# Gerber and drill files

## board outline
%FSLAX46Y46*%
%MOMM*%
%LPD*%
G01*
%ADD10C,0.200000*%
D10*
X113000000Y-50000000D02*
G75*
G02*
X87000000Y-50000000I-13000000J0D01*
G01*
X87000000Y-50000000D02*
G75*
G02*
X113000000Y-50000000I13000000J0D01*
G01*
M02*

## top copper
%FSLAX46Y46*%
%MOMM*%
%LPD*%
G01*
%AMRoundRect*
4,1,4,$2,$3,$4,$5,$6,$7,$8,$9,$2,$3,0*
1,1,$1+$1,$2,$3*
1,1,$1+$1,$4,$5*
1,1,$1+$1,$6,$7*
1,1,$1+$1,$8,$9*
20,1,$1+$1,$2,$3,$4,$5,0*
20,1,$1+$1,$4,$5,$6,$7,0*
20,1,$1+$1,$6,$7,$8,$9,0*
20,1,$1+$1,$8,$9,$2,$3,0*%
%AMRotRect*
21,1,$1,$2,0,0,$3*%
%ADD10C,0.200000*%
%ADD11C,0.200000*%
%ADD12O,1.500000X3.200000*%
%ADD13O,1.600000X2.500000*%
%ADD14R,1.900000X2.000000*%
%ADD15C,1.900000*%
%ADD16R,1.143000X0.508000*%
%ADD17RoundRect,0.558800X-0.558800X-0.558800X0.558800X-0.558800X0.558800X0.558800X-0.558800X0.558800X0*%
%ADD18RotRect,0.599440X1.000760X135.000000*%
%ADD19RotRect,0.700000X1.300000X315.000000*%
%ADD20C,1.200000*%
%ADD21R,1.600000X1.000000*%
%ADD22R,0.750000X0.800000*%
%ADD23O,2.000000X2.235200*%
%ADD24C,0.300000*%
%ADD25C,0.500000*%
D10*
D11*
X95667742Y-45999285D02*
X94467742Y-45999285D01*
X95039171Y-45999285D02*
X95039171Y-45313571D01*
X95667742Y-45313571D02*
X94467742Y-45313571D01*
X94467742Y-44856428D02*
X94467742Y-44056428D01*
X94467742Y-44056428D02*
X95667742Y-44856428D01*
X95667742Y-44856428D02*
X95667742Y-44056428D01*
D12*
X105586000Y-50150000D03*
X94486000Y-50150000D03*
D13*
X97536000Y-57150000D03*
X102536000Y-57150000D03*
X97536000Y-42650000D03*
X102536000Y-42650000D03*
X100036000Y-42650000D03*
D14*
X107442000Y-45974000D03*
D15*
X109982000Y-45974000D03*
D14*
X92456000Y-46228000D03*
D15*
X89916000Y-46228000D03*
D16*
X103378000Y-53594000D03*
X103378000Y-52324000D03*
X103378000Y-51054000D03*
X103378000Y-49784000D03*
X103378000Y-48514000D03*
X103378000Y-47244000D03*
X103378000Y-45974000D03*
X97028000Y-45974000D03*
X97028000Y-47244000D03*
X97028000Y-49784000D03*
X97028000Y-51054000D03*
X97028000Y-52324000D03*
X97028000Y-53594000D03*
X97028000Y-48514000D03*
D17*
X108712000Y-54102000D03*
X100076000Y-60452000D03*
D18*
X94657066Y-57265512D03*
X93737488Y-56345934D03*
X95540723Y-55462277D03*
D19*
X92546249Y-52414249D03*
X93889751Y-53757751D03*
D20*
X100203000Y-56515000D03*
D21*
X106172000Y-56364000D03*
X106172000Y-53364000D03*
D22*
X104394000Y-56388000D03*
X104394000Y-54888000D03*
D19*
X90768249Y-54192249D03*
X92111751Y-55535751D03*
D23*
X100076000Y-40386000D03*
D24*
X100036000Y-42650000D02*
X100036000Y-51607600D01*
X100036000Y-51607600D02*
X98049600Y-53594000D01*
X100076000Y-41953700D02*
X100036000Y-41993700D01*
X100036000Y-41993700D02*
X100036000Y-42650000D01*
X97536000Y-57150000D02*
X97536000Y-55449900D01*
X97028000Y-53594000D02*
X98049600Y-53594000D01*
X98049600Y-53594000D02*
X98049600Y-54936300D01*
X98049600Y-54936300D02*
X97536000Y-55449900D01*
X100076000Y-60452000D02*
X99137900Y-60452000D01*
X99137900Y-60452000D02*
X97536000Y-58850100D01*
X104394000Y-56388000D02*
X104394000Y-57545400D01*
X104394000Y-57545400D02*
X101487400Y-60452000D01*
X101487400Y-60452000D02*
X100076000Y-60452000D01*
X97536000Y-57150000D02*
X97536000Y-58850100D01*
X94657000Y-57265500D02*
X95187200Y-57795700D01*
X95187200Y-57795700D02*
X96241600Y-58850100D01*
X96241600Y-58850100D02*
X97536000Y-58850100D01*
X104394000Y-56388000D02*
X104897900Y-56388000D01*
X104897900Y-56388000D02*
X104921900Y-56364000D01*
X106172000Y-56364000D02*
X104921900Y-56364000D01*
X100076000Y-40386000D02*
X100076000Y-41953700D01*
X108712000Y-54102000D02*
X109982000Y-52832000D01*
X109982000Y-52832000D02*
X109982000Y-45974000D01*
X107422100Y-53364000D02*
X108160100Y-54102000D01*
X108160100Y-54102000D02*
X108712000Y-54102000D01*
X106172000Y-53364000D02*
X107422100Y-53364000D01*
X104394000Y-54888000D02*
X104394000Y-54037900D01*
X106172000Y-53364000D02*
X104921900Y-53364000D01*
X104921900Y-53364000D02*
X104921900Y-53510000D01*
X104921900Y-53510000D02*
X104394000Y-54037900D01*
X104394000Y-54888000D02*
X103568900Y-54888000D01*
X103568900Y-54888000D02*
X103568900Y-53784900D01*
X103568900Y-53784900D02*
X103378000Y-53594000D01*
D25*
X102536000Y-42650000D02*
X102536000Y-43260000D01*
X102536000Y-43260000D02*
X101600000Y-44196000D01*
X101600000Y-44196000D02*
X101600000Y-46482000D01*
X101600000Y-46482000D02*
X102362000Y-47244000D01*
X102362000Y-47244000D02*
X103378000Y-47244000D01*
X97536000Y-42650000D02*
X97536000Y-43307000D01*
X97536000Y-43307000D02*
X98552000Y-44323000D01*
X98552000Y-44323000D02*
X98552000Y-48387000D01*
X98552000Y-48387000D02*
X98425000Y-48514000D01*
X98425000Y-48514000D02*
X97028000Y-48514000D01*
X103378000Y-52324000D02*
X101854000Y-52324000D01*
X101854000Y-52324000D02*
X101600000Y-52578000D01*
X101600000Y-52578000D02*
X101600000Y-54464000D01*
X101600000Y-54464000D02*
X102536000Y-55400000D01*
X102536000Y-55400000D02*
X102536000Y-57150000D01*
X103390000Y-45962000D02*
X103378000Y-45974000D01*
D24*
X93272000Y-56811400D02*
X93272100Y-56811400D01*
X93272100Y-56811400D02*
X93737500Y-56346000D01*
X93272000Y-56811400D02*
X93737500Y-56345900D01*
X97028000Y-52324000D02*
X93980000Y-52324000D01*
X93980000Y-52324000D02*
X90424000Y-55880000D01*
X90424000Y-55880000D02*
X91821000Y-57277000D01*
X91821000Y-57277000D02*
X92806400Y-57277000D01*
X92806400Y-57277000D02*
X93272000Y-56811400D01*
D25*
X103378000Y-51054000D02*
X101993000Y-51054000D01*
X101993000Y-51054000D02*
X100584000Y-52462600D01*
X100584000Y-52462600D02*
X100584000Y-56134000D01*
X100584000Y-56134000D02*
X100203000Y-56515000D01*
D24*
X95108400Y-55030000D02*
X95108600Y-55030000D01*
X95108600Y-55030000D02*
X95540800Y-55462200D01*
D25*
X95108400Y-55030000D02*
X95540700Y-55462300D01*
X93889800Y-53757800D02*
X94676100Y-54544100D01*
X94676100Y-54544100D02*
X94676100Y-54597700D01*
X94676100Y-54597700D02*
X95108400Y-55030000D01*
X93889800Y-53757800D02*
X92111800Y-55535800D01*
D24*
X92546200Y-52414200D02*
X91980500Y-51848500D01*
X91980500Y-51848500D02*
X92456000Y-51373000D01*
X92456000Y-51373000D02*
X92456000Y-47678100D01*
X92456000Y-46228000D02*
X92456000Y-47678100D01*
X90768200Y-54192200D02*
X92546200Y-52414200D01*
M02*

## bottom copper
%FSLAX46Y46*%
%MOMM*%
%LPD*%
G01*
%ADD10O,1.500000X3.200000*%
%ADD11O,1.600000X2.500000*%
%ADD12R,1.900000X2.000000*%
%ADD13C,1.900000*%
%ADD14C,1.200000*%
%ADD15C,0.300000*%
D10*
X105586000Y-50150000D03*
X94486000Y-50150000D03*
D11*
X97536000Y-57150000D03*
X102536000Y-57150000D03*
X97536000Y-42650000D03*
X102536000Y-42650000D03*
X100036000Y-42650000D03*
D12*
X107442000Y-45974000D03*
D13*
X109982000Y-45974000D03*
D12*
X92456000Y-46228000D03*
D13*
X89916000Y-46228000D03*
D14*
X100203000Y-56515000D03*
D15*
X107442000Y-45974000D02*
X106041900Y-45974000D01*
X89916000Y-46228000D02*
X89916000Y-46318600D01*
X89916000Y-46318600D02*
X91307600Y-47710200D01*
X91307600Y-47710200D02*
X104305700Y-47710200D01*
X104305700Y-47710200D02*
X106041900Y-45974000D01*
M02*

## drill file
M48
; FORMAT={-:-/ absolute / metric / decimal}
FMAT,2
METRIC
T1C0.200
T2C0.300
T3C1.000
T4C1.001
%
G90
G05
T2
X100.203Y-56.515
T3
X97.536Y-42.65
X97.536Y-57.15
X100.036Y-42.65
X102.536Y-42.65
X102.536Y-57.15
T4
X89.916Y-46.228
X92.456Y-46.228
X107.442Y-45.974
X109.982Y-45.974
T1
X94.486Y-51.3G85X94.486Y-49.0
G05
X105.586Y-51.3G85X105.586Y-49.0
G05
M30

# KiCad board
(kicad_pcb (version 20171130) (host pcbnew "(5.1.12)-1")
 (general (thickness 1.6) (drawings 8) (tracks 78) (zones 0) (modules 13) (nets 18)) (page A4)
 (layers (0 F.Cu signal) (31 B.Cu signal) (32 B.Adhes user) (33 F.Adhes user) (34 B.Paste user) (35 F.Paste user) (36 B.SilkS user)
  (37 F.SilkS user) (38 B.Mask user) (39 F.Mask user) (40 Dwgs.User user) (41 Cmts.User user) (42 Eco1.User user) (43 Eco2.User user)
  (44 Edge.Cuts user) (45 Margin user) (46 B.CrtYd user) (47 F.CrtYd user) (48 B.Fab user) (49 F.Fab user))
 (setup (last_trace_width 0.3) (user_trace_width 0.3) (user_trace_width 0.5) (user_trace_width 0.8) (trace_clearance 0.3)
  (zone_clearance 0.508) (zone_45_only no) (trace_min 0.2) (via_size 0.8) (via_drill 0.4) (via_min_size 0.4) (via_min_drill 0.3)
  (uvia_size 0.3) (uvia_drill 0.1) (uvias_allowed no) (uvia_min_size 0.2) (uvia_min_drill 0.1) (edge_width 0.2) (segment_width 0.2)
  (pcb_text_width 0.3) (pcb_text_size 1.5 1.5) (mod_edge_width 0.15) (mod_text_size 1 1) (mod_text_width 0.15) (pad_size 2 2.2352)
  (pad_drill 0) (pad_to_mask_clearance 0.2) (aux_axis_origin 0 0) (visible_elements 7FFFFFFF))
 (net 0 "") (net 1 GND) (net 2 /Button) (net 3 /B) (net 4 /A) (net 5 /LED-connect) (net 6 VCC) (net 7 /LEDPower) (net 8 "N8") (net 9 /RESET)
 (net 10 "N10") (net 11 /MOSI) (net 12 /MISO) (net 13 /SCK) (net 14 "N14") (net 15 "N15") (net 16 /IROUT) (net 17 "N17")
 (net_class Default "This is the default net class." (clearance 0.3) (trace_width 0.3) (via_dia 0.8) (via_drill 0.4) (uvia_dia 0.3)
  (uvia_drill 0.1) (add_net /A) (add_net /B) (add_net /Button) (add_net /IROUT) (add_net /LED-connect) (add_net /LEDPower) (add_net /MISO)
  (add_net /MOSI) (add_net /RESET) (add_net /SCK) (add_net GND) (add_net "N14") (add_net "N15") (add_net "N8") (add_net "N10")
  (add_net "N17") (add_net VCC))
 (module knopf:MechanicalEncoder (layer B.Cu) (at 100.036 50.15 180)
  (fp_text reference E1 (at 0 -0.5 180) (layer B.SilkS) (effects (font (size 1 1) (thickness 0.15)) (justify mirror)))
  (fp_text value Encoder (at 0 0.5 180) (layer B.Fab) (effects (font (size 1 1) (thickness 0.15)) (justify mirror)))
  (pad 6 thru_hole oval (at -5.55 0 180) (size 1.5 3.2) (drill oval 0.2 2.5) (layers *.Cu *.Mask))
  (pad 6 thru_hole oval (at 5.55 0 180) (size 1.5 3.2) (drill oval 0.2 2.5) (layers *.Cu *.Mask))
  (pad 5 thru_hole oval (at 2.5 -7 180) (size 1.6 2.5) (drill 1) (layers *.Cu *.Mask) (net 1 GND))
  (pad 4 thru_hole oval (at -2.5 -7 180) (size 1.6 2.5) (drill 1) (layers *.Cu *.Mask) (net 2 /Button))
  (pad 3 thru_hole oval (at 2.5 7.5 180) (size 1.6 2.5) (drill 1) (layers *.Cu *.Mask) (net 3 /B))
  (pad 1 thru_hole oval (at -2.5 7.5 180) (size 1.6 2.5) (drill 1) (layers *.Cu *.Mask) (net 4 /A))
  (pad 2 thru_hole oval (at 0 7.5 180) (size 1.6 2.5) (drill 1) (layers *.Cu *.Mask) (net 1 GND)))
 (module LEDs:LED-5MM (layer F.Cu) (at 107.442 45.974)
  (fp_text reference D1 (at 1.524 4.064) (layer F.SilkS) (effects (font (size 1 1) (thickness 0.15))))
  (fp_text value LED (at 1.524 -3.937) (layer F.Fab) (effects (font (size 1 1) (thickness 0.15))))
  (pad 1 thru_hole rect (at 0 0 90) (size 2 1.9) (drill 1.00076) (layers *.Cu *.Mask F.SilkS) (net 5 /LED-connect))
  (pad 2 thru_hole circle (at 2.54 0) (size 1.9 1.9) (drill 1.00076) (layers *.Cu *.Mask F.SilkS) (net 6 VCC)))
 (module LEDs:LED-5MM (layer F.Cu) (at 92.456 46.228 180)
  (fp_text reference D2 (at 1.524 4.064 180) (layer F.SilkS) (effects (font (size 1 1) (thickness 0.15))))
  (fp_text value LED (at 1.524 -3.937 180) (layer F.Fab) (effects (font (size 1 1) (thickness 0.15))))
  (pad 1 thru_hole rect (at 0 0 270) (size 2 1.9) (drill 1.00076) (layers *.Cu *.Mask F.SilkS) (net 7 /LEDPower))
  (pad 2 thru_hole circle (at 2.54 0 180) (size 1.9 1.9) (drill 1.00076) (layers *.Cu *.Mask F.SilkS) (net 5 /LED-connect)))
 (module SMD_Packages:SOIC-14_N (layer F.Cu) (at 100.076 49.784 90)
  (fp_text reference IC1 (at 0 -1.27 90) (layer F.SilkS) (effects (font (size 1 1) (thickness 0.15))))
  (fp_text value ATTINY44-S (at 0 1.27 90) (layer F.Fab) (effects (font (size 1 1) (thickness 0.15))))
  (pad 1 smd rect (at -3.81 3.302 90) (size 0.508 1.143) (layers F.Cu F.Paste F.Mask) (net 6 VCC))
  (pad 2 smd rect (at -2.54 3.302 90) (size 0.508 1.143) (layers F.Cu F.Paste F.Mask) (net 2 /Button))
  (pad 3 smd rect (at -1.27 3.302 90) (size 0.508 1.143) (layers F.Cu F.Paste F.Mask) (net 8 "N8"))
  (pad 4 smd rect (at 0 3.302 90) (size 0.508 1.143) (layers F.Cu F.Paste F.Mask) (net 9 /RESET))
  (pad 5 smd rect (at 1.27 3.302 90) (size 0.508 1.143) (layers F.Cu F.Paste F.Mask) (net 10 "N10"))
  (pad 6 smd rect (at 2.54 3.302 90) (size 0.508 1.143) (layers F.Cu F.Paste F.Mask) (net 4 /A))
  (pad 7 smd rect (at 3.81 3.302 90) (size 0.508 1.143) (layers F.Cu F.Paste F.Mask) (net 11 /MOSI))
  (pad 8 smd rect (at 3.81 -3.048 90) (size 0.508 1.143) (layers F.Cu F.Paste F.Mask) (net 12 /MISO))
  (pad 9 smd rect (at 2.54 -3.048 90) (size 0.508 1.143) (layers F.Cu F.Paste F.Mask) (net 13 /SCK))
  (pad 11 smd rect (at 0 -3.048 90) (size 0.508 1.143) (layers F.Cu F.Paste F.Mask) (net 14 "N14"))
  (pad 12 smd rect (at -1.27 -3.048 90) (size 0.508 1.143) (layers F.Cu F.Paste F.Mask) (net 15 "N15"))
  (pad 13 smd rect (at -2.54 -3.048 90) (size 0.508 1.143) (layers F.Cu F.Paste F.Mask) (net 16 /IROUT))
  (pad 14 smd rect (at -3.81 -3.048 90) (size 0.508 1.143) (layers F.Cu F.Paste F.Mask) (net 1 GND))
  (pad 10 smd rect (at 1.27 -3.048 90) (size 0.508 1.143) (layers F.Cu F.Paste F.Mask) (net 3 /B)))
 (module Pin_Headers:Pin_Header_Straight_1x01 (layer F.Cu) (at 108.712 54.102)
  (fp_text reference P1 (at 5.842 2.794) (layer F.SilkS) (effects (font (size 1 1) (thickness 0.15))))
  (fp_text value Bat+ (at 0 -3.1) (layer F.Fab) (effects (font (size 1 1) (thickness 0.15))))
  (pad 1 smd roundrect (at 0 0) (size 2.2352 2.2352) (layers F.Cu F.Paste F.Mask) (roundrect_rratio 0.25) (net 6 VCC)))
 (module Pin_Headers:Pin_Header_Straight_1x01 (layer F.Cu) (at 100.076 60.452)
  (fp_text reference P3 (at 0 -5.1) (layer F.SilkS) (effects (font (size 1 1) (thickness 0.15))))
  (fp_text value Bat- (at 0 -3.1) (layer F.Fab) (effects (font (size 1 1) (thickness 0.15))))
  (pad 1 smd roundrect (at 0 0) (size 2.2352 2.2352) (layers F.Cu F.Paste F.Mask) (roundrect_rratio 0.25) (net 1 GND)))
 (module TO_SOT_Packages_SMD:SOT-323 (layer F.Cu) (at 94.869 56.134 135)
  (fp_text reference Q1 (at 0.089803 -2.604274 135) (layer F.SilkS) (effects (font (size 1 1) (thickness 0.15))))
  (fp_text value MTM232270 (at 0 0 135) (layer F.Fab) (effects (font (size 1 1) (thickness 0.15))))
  (pad 2 smd rect (at -0.65024 -0.94996 135) (size 0.59944 1.00076) (layers F.Cu F.Paste F.Mask) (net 1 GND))
  (pad 1 smd rect (at 0.65024 -0.94996 135) (size 0.59944 1.00076) (layers F.Cu F.Paste F.Mask) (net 16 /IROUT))
  (pad 3 smd rect (at 0 0.94996 135) (size 0.59944 1.00076) (layers F.Cu F.Paste F.Mask) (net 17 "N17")))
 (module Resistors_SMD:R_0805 (layer F.Cu) (at 93.218 53.086 315)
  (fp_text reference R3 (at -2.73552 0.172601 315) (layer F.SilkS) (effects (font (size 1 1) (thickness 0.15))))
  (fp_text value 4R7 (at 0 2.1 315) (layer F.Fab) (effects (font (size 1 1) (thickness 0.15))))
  (pad 1 smd rect (at -0.949999 0 315) (size 0.7 1.3) (layers F.Cu F.Paste F.Mask) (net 7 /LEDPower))
  (pad 2 smd rect (at 0.949999 0 315) (size 0.7 1.3) (layers F.Cu F.Paste F.Mask) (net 17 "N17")))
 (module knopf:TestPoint (layer F.Cu) (at 100.203 56.515)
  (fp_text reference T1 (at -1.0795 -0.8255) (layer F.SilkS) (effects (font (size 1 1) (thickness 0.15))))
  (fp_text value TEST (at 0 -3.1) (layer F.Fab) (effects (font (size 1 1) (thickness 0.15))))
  (pad 1 thru_hole circle (at 0 0) (size 1.2 1.2) (drill 0.3) (layers *.Cu *.Mask F.SilkS) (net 8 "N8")))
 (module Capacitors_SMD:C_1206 (layer F.Cu) (at 106.172 54.864 270)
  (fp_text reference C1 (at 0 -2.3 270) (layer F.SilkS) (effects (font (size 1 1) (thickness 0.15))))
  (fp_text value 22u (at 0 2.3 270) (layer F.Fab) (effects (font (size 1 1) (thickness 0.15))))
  (pad 2 smd rect (at 1.5 0 270) (size 1 1.6) (layers F.Cu F.Paste F.Mask) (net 1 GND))
  (pad 1 smd rect (at -1.5 0 270) (size 1 1.6) (layers F.Cu F.Paste F.Mask) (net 6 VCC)))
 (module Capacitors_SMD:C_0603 (layer F.Cu) (at 104.394 55.638 270)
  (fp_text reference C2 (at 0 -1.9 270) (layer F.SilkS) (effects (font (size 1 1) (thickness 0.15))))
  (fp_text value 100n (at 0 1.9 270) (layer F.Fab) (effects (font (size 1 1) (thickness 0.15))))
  (pad 2 smd rect (at 0.75 0 270) (size 0.8 0.75) (layers F.Cu F.Paste F.Mask) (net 1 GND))
  (pad 1 smd rect (at -0.75 0 270) (size 0.8 0.75) (layers F.Cu F.Paste F.Mask) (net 6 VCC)))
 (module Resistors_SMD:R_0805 (layer F.Cu) (at 91.44 54.864 315)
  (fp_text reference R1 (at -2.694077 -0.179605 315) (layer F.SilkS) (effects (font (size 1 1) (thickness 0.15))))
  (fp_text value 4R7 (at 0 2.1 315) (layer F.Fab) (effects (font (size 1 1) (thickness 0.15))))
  (pad 1 smd rect (at -0.949999 0 315) (size 0.7 1.3) (layers F.Cu F.Paste F.Mask) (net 7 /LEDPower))
  (pad 2 smd rect (at 0.949999 0 315) (size 0.7 1.3) (layers F.Cu F.Paste F.Mask) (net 17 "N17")))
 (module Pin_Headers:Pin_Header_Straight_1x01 (layer F.Cu) (at 100.076 40.386)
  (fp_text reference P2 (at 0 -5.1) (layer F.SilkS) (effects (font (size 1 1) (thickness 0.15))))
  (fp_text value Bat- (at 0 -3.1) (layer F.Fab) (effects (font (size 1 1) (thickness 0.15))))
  (pad 1 smd oval (at 0 0) (size 2 2.2352) (layers F.Cu F.Paste F.Mask) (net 1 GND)))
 (gr_circle (center 100 50) (end 113 50) (layer Edge.Cuts) (width 0.2))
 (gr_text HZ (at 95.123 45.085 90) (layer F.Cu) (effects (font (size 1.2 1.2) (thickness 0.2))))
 (segment (start 100.036 42.65) (end 100.036 51.6076) (width 0.3) (layer F.Cu) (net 1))
 (segment (start 100.036 51.6076) (end 98.0496 53.594) (width 0.3) (layer F.Cu) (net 1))
 (segment (start 100.076 41.9537) (end 100.036 41.9937) (width 0.3) (layer F.Cu) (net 1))
 (segment (start 100.036 41.9937) (end 100.036 42.65) (width 0.3) (layer F.Cu) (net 1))
 (segment (start 97.536 57.15) (end 97.536 55.4499) (width 0.3) (layer F.Cu) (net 1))
 (segment (start 97.028 53.594) (end 98.0496 53.594) (width 0.3) (layer F.Cu) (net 1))
 (segment (start 98.0496 53.594) (end 98.0496 54.9363) (width 0.3) (layer F.Cu) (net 1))
 (segment (start 98.0496 54.9363) (end 97.536 55.4499) (width 0.3) (layer F.Cu) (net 1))
 (segment (start 100.076 60.452) (end 99.1379 60.452) (width 0.3) (layer F.Cu) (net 1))
 (segment (start 99.1379 60.452) (end 97.536 58.8501) (width 0.3) (layer F.Cu) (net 1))
 (segment (start 104.394 56.388) (end 104.394 57.5454) (width 0.3) (layer F.Cu) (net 1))
 (segment (start 104.394 57.5454) (end 101.4874 60.452) (width 0.3) (layer F.Cu) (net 1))
 (segment (start 101.4874 60.452) (end 100.076 60.452) (width 0.3) (layer F.Cu) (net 1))
 (segment (start 97.536 57.15) (end 97.536 58.8501) (width 0.3) (layer F.Cu) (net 1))
 (segment (start 94.657 57.2655) (end 95.1872 57.7957) (width 0.3) (layer F.Cu) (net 1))
 (segment (start 95.1872 57.7957) (end 96.2416 58.8501) (width 0.3) (layer F.Cu) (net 1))
 (segment (start 96.2416 58.8501) (end 97.536 58.8501) (width 0.3) (layer F.Cu) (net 1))
 (segment (start 104.394 56.388) (end 104.8979 56.388) (width 0.3) (layer F.Cu) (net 1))
 (segment (start 104.8979 56.388) (end 104.9219 56.364) (width 0.3) (layer F.Cu) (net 1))
 (segment (start 106.172 56.364) (end 104.9219 56.364) (width 0.3) (layer F.Cu) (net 1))
 (segment (start 100.076 40.386) (end 100.076 41.9537) (width 0.3) (layer F.Cu) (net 1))
 (segment (start 108.712 54.102) (end 109.982 52.832) (width 0.3) (layer F.Cu) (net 6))
 (segment (start 109.982 52.832) (end 109.982 45.974) (width 0.3) (layer F.Cu) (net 6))
 (segment (start 107.4221 53.364) (end 108.1601 54.102) (width 0.3) (layer F.Cu) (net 6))
 (segment (start 108.1601 54.102) (end 108.712 54.102) (width 0.3) (layer F.Cu) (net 6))
 (segment (start 106.172 53.364) (end 107.4221 53.364) (width 0.3) (layer F.Cu) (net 6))
 (segment (start 104.394 54.888) (end 104.394 54.0379) (width 0.3) (layer F.Cu) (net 6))
 (segment (start 106.172 53.364) (end 104.9219 53.364) (width 0.3) (layer F.Cu) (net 6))
 (segment (start 104.9219 53.364) (end 104.9219 53.51) (width 0.3) (layer F.Cu) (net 6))
 (segment (start 104.9219 53.51) (end 104.394 54.0379) (width 0.3) (layer F.Cu) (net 6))
 (segment (start 104.394 54.888) (end 103.5689 54.888) (width 0.3) (layer F.Cu) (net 6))
 (segment (start 103.5689 54.888) (end 103.5689 53.7849) (width 0.3) (layer F.Cu) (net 6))
 (segment (start 103.5689 53.7849) (end 103.378 53.594) (width 0.3) (layer F.Cu) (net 6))
 (segment (start 102.536 42.65) (end 102.536 43.26) (width 0.5) (layer F.Cu) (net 4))
 (segment (start 102.536 43.26) (end 101.6 44.196) (width 0.5) (layer F.Cu) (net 4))
 (segment (start 101.6 44.196) (end 101.6 46.482) (width 0.5) (layer F.Cu) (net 4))
 (segment (start 101.6 46.482) (end 102.362 47.244) (width 0.5) (layer F.Cu) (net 4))
 (segment (start 102.362 47.244) (end 103.378 47.244) (width 0.5) (layer F.Cu) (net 4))
 (segment (start 97.536 42.65) (end 97.536 43.307) (width 0.5) (layer F.Cu) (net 3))
 (segment (start 97.536 43.307) (end 98.552 44.323) (width 0.5) (layer F.Cu) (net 3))
 (segment (start 98.552 44.323) (end 98.552 48.387) (width 0.5) (layer F.Cu) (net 3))
 (segment (start 98.552 48.387) (end 98.425 48.514) (width 0.5) (layer F.Cu) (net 3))
 (segment (start 98.425 48.514) (end 97.028 48.514) (width 0.5) (layer F.Cu) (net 3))
 (segment (start 103.378 52.324) (end 101.854 52.324) (width 0.5) (layer F.Cu) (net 2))
 (segment (start 101.854 52.324) (end 101.6 52.578) (width 0.5) (layer F.Cu) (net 2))
 (segment (start 101.6 52.578) (end 101.6 54.464) (width 0.5) (layer F.Cu) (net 2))
 (segment (start 101.6 54.464) (end 102.536 55.4) (width 0.5) (layer F.Cu) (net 2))
 (segment (start 102.536 55.4) (end 102.536 57.15) (width 0.5) (layer F.Cu) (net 2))
 (segment (start 103.39 45.962) (end 103.378 45.974) (width 0.5) (layer F.Cu) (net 11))
 (segment (start 93.272 56.8114) (end 93.2721 56.8114) (width 0.3) (layer F.Cu) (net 16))
 (segment (start 93.2721 56.8114) (end 93.7375 56.346) (width 0.3) (layer F.Cu) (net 16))
 (segment (start 93.272 56.8114) (end 93.7375 56.3459) (width 0.3) (layer F.Cu) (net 16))
 (segment (start 97.028 52.324) (end 93.98 52.324) (width 0.3) (layer F.Cu) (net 16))
 (segment (start 93.98 52.324) (end 90.424 55.88) (width 0.3) (layer F.Cu) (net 16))
 (segment (start 90.424 55.88) (end 91.821 57.277) (width 0.3) (layer F.Cu) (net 16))
 (segment (start 91.821 57.277) (end 92.8064 57.277) (width 0.3) (layer F.Cu) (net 16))
 (segment (start 92.8064 57.277) (end 93.272 56.8114) (width 0.3) (layer F.Cu) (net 16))
 (segment (start 103.378 51.054) (end 101.993 51.054) (width 0.5) (layer F.Cu) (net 8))
 (segment (start 101.993 51.054) (end 100.584 52.4626) (width 0.5) (layer F.Cu) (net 8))
 (segment (start 100.584 52.4626) (end 100.584 56.134) (width 0.5) (layer F.Cu) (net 8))
 (segment (start 100.584 56.134) (end 100.203 56.515) (width 0.5) (layer F.Cu) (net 8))
 (segment (start 95.1084 55.03) (end 95.1086 55.03) (width 0.3) (layer F.Cu) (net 17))
 (segment (start 95.1086 55.03) (end 95.5408 55.4622) (width 0.3) (layer F.Cu) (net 17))
 (segment (start 95.1084 55.03) (end 95.5407 55.4623) (width 0.5) (layer F.Cu) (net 17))
 (segment (start 93.8898 53.7578) (end 94.6761 54.5441) (width 0.5) (layer F.Cu) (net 17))
 (segment (start 94.6761 54.5441) (end 94.6761 54.5977) (width 0.5) (layer F.Cu) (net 17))
 (segment (start 94.6761 54.5977) (end 95.1084 55.03) (width 0.5) (layer F.Cu) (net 17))
 (segment (start 93.8898 53.7578) (end 92.1118 55.5358) (width 0.5) (layer F.Cu) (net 17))
 (segment (start 107.442 45.974) (end 106.0419 45.974) (width 0.3) (layer B.Cu) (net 5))
 (segment (start 89.916 46.228) (end 89.916 46.3186) (width 0.3) (layer B.Cu) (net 5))
 (segment (start 89.916 46.3186) (end 91.3076 47.7102) (width 0.3) (layer B.Cu) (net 5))
 (segment (start 91.3076 47.7102) (end 104.3057 47.7102) (width 0.3) (layer B.Cu) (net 5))
 (segment (start 104.3057 47.7102) (end 106.0419 45.974) (width 0.3) (layer B.Cu) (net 5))
 (segment (start 92.5462 52.4142) (end 91.9805 51.8485) (width 0.3) (layer F.Cu) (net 7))
 (segment (start 91.9805 51.8485) (end 92.456 51.373) (width 0.3) (layer F.Cu) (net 7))
 (segment (start 92.456 51.373) (end 92.456 47.6781) (width 0.3) (layer F.Cu) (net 7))
 (segment (start 92.456 46.228) (end 92.456 47.6781) (width 0.3) (layer F.Cu) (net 7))
 (segment (start 90.7682 54.1922) (end 92.5462 52.4142) (width 0.3) (layer F.Cu) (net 7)))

